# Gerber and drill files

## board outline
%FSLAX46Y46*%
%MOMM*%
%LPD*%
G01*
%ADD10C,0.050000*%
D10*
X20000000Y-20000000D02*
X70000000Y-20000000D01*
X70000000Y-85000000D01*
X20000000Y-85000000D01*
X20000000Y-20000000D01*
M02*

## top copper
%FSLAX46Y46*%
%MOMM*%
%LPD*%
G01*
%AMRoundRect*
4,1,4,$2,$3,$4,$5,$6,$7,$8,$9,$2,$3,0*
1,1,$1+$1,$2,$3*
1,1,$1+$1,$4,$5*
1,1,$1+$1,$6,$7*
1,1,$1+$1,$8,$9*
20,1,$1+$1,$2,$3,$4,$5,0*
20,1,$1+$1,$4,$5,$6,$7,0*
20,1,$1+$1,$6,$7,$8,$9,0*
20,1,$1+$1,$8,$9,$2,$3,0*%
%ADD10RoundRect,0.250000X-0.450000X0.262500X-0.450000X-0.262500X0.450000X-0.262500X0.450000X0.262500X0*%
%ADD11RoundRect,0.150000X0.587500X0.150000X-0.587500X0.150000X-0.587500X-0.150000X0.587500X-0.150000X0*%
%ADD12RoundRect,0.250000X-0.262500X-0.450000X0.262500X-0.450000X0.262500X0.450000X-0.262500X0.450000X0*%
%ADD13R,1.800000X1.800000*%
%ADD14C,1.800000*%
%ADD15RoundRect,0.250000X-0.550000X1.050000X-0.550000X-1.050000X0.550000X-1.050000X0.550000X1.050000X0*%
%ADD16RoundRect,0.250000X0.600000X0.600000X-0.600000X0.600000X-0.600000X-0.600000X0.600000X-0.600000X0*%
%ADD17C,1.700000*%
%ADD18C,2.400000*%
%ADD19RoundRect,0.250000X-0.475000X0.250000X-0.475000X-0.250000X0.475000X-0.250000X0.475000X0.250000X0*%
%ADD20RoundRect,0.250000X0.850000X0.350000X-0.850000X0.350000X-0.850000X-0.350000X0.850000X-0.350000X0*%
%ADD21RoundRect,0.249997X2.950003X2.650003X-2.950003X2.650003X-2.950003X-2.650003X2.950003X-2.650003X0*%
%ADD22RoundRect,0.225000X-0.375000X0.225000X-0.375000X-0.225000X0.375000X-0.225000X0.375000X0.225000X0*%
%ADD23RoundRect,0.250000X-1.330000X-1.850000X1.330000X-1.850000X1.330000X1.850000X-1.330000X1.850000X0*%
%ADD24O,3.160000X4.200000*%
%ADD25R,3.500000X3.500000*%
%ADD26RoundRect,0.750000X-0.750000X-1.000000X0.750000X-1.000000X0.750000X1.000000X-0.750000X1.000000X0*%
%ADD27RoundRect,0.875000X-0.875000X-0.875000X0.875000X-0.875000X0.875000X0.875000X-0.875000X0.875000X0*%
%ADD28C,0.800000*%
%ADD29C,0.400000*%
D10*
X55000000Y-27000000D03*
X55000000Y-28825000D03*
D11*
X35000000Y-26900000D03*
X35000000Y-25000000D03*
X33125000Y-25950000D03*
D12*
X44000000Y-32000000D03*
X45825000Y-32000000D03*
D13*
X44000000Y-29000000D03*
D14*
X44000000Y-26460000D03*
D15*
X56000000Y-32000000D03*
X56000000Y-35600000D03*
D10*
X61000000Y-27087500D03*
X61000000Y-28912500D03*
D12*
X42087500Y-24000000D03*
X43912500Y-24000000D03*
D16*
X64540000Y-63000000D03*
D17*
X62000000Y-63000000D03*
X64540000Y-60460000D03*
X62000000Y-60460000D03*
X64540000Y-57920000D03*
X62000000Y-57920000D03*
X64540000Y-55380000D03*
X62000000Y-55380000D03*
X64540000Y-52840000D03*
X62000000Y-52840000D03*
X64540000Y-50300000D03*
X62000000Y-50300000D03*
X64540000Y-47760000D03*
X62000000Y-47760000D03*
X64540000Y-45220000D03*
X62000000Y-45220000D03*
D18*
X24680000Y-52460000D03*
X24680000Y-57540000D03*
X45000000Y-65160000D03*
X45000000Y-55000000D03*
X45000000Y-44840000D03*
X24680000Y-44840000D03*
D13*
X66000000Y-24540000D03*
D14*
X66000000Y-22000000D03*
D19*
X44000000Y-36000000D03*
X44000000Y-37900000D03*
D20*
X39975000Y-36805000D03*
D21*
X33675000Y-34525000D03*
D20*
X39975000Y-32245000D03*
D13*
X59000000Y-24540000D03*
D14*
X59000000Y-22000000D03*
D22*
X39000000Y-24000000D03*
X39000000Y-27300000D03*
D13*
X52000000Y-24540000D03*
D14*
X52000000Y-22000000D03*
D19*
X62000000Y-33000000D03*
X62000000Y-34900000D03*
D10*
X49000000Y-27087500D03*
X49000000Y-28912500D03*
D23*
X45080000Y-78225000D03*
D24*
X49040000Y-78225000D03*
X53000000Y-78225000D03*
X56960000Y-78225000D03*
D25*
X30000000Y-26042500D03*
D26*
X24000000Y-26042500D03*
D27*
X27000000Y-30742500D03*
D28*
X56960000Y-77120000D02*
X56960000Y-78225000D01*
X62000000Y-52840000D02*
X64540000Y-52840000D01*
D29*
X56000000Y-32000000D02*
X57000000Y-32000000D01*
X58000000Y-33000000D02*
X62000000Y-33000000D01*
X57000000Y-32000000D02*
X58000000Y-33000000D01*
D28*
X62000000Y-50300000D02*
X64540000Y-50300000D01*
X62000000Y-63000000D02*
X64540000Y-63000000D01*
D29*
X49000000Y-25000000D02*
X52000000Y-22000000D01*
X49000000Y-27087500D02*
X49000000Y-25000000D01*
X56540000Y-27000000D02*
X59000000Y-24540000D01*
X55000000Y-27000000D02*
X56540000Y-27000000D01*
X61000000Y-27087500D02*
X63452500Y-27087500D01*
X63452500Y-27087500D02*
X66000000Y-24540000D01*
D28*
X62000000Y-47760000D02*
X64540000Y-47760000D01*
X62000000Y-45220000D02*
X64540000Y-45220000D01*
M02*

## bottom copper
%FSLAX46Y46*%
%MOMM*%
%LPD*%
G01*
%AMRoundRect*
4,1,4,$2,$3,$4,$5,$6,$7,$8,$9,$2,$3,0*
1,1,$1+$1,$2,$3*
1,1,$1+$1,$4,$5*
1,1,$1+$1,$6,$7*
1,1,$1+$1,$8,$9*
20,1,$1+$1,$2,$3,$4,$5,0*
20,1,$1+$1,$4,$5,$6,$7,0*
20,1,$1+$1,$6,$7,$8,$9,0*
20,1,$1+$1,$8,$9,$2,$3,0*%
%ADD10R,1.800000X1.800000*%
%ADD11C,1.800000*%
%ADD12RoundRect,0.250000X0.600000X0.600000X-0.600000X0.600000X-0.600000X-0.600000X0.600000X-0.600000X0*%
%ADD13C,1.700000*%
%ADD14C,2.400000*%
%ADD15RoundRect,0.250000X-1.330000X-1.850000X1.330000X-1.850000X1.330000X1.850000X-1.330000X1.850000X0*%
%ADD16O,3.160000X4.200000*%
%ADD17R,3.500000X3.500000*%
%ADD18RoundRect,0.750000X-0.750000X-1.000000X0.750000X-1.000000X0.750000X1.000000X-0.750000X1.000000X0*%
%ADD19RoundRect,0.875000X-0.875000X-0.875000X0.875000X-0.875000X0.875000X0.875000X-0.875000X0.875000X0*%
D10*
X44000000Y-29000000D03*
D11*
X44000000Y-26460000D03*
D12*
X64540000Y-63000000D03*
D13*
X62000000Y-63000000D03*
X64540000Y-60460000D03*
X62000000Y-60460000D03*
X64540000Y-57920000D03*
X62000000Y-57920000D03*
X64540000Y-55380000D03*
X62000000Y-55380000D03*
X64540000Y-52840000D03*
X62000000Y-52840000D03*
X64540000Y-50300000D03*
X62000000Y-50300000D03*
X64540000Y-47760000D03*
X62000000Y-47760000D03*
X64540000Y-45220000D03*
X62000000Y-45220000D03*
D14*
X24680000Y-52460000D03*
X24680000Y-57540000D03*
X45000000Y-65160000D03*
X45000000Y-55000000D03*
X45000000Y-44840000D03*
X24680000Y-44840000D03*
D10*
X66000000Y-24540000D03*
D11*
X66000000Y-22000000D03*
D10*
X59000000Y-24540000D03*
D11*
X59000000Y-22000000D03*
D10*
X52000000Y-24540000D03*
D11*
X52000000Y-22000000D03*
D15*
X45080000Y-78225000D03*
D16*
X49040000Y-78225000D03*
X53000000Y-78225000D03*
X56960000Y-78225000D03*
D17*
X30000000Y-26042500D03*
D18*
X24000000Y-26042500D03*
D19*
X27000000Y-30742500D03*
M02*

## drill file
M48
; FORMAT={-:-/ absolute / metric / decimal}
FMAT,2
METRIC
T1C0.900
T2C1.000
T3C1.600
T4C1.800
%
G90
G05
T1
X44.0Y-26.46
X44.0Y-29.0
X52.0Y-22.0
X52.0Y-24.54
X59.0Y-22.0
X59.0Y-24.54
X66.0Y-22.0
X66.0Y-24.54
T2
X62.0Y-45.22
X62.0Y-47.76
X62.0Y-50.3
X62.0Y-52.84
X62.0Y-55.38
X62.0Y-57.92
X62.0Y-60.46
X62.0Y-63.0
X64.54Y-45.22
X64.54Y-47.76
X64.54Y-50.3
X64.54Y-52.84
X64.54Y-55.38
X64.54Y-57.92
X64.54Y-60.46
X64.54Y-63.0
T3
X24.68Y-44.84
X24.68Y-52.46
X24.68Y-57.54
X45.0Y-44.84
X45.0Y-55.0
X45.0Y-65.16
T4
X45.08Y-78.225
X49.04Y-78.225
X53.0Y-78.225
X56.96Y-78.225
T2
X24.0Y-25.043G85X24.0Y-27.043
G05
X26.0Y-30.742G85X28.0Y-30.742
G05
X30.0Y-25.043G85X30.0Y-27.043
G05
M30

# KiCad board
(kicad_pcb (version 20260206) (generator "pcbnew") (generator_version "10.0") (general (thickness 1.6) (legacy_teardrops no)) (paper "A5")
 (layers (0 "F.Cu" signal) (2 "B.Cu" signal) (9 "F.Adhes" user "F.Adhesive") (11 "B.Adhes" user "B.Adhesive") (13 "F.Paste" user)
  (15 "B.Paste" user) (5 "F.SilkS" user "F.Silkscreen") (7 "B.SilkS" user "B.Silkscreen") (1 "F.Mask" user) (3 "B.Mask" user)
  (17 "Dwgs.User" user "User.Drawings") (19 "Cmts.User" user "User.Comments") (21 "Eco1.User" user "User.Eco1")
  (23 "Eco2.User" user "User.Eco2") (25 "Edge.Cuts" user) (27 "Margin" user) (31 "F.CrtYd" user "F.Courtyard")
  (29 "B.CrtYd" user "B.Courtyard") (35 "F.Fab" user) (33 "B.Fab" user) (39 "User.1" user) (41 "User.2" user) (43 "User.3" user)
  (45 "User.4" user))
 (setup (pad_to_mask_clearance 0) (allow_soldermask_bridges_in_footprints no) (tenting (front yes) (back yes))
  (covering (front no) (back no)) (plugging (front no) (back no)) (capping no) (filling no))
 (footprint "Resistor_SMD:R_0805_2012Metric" (layer "F.Cu") (at 55 27.9125 -90)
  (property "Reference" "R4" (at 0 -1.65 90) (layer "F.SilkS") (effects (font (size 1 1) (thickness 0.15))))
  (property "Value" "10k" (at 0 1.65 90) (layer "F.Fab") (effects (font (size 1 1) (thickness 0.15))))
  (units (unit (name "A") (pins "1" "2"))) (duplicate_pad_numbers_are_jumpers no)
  (pad "1" smd roundrect (at -0.9125 0 270) (size 1.025 1.4) (layers "F.Cu" "F.Mask" "F.Paste") (roundrect_rratio 0.243902)
   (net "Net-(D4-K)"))
  (pad "2" smd roundrect (at 0.9125 0 270) (size 1.025 1.4) (layers "F.Cu" "F.Mask" "F.Paste") (roundrect_rratio 0.243902) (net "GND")))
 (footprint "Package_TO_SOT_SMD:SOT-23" (layer "F.Cu") (at 34.0625 25.95 180)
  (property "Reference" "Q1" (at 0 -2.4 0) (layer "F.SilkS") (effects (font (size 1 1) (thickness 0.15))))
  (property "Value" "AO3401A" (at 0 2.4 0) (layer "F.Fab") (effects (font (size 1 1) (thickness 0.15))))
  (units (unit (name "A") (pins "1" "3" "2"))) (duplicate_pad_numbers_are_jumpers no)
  (pad "1" smd roundrect (at -0.9375 -0.95 180) (size 1.475 0.6) (layers "F.Cu" "F.Mask" "F.Paste") (roundrect_rratio 0.25)
   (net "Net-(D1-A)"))
  (pad "2" smd roundrect (at -0.9375 0.95 180) (size 1.475 0.6) (layers "F.Cu" "F.Mask" "F.Paste") (roundrect_rratio 0.25)
   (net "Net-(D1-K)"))
  (pad "3" smd roundrect (at 0.9375 0 180) (size 1.475 0.6) (layers "F.Cu" "F.Mask" "F.Paste") (roundrect_rratio 0.25) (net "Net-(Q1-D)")))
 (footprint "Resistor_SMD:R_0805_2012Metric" (layer "F.Cu") (at 44.9125 32)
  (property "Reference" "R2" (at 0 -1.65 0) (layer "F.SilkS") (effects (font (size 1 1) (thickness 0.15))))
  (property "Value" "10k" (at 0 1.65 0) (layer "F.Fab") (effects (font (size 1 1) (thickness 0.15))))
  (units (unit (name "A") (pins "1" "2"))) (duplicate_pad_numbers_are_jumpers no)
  (pad "1" smd roundrect (at -0.9125 0) (size 1.025 1.4) (layers "F.Cu" "F.Mask" "F.Paste") (roundrect_rratio 0.243902) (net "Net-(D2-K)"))
  (pad "2" smd roundrect (at 0.9125 0) (size 1.025 1.4) (layers "F.Cu" "F.Mask" "F.Paste") (roundrect_rratio 0.243902) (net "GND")))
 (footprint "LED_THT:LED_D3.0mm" (layer "F.Cu") (at 44 29 90)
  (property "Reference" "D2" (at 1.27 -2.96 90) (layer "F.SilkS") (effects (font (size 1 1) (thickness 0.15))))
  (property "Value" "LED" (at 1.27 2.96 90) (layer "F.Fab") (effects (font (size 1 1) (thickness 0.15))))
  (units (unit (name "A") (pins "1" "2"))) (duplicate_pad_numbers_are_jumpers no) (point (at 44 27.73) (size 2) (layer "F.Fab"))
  (pad "1" thru_hole rect (at 0 0 90) (size 1.8 1.8) (drill 0.9) (layers "*.Cu" "*.Mask") (remove_unused_layers no) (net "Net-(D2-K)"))
  (pad "2" thru_hole circle (at 2.54 0 90) (size 1.8 1.8) (drill 0.9) (layers "*.Cu" "*.Mask") (remove_unused_layers no) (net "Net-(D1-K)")))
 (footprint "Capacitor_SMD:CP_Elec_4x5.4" (layer "F.Cu") (at 56 33.8 -90)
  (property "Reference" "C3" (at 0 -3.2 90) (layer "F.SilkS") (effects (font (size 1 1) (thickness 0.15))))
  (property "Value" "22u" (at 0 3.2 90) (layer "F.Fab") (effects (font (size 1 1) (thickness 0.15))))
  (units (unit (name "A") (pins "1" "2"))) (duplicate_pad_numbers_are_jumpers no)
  (pad "1" smd roundrect (at -1.8 0 270) (size 2.6 1.6) (layers "F.Cu" "F.Mask" "F.Paste") (roundrect_rratio 0.15625) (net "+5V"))
  (pad "2" smd roundrect (at 1.8 0 270) (size 2.6 1.6) (layers "F.Cu" "F.Mask" "F.Paste") (roundrect_rratio 0.15625) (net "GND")))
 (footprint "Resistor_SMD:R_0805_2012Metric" (layer "F.Cu") (at 61 28 -90)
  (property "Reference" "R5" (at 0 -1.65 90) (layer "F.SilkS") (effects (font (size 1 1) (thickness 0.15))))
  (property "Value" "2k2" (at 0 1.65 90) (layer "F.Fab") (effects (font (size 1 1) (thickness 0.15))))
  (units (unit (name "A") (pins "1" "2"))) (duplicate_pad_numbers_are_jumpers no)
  (pad "1" smd roundrect (at -0.9125 0 270) (size 1.025 1.4) (layers "F.Cu" "F.Mask" "F.Paste") (roundrect_rratio 0.243902)
   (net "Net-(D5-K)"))
  (pad "2" smd roundrect (at 0.9125 0 270) (size 1.025 1.4) (layers "F.Cu" "F.Mask" "F.Paste") (roundrect_rratio 0.243902) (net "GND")))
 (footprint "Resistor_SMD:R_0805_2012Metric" (layer "F.Cu") (at 43 24)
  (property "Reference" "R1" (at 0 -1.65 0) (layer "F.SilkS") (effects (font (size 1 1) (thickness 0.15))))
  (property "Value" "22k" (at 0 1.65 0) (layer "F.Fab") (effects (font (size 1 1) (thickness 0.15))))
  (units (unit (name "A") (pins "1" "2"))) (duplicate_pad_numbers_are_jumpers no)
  (pad "1" smd roundrect (at -0.9125 0) (size 1.025 1.4) (layers "F.Cu" "F.Mask" "F.Paste") (roundrect_rratio 0.243902) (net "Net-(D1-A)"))
  (pad "2" smd roundrect (at 0.9125 0) (size 1.025 1.4) (layers "F.Cu" "F.Mask" "F.Paste") (roundrect_rratio 0.243902) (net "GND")))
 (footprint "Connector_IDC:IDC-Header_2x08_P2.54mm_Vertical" (layer "F.Cu") (at 64.54 63 180)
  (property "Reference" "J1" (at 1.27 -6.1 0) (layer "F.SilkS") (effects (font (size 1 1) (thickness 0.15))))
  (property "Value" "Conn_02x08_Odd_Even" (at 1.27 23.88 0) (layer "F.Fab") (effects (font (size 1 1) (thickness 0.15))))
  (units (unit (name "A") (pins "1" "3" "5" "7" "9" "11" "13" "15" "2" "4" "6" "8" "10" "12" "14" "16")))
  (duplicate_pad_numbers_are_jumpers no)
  (pad "1" thru_hole roundrect (at 0 0 180) (size 1.7 1.7) (drill 1) (layers "*.Cu" "*.Mask") (remove_unused_layers no)
   (roundrect_rratio 0.147059) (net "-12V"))
  (pad "2" thru_hole circle (at 2.54 0 180) (size 1.7 1.7) (drill 1) (layers "*.Cu" "*.Mask") (remove_unused_layers no) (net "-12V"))
  (pad "3" thru_hole circle (at 0 2.54 180) (size 1.7 1.7) (drill 1) (layers "*.Cu" "*.Mask") (remove_unused_layers no) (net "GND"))
  (pad "4" thru_hole circle (at 2.54 2.54 180) (size 1.7 1.7) (drill 1) (layers "*.Cu" "*.Mask") (remove_unused_layers no) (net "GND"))
  (pad "5" thru_hole circle (at 0 5.08 180) (size 1.7 1.7) (drill 1) (layers "*.Cu" "*.Mask") (remove_unused_layers no) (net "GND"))
  (pad "6" thru_hole circle (at 2.54 5.08 180) (size 1.7 1.7) (drill 1) (layers "*.Cu" "*.Mask") (remove_unused_layers no) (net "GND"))
  (pad "7" thru_hole circle (at 0 7.62 180) (size 1.7 1.7) (drill 1) (layers "*.Cu" "*.Mask") (remove_unused_layers no) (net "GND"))
  (pad "8" thru_hole circle (at 2.54 7.62 180) (size 1.7 1.7) (drill 1) (layers "*.Cu" "*.Mask") (remove_unused_layers no) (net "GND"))
  (pad "9" thru_hole circle (at 0 10.16 180) (size 1.7 1.7) (drill 1) (layers "*.Cu" "*.Mask") (remove_unused_layers no) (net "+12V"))
  (pad "10" thru_hole circle (at 2.54 10.16 180) (size 1.7 1.7) (drill 1) (layers "*.Cu" "*.Mask") (remove_unused_layers no) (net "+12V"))
  (pad "11" thru_hole circle (at 0 12.7 180) (size 1.7 1.7) (drill 1) (layers "*.Cu" "*.Mask") (remove_unused_layers no) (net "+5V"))
  (pad "12" thru_hole circle (at 2.54 12.7 180) (size 1.7 1.7) (drill 1) (layers "*.Cu" "*.Mask") (remove_unused_layers no) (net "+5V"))
  (pad "13" thru_hole circle (at 0 15.24 180) (size 1.7 1.7) (drill 1) (layers "*.Cu" "*.Mask") (remove_unused_layers no) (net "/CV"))
  (pad "14" thru_hole circle (at 2.54 15.24 180) (size 1.7 1.7) (drill 1) (layers "*.Cu" "*.Mask") (remove_unused_layers no) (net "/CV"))
  (pad "15" thru_hole circle (at 0 17.78 180) (size 1.7 1.7) (drill 1) (layers "*.Cu" "*.Mask") (remove_unused_layers no) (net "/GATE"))
  (pad "16" thru_hole circle (at 2.54 17.78 180) (size 1.7 1.7) (drill 1) (layers "*.Cu" "*.Mask") (remove_unused_layers no) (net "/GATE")))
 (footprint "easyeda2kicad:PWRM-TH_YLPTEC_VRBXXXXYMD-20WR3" (layer "F.Cu") (at 34.84 55)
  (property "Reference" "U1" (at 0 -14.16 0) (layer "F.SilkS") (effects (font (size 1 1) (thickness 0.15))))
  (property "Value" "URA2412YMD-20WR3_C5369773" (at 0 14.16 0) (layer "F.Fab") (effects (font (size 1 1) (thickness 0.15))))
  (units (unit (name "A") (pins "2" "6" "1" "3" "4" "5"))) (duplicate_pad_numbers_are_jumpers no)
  (pad "1" thru_hole circle (at -10.16 -2.54 90) (size 2.4 2.4) (drill 1.599996) (layers "*.Cu" "*.Mask") (remove_unused_layers no)
   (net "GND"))
  (pad "2" thru_hole circle (at -10.16 2.54 90) (size 2.4 2.4) (drill 1.599996) (layers "*.Cu" "*.Mask") (remove_unused_layers no)
   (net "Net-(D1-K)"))
  (pad "3" thru_hole circle (at 10.16 10.16 90) (size 2.4 2.4) (drill 1.599996) (layers "*.Cu" "*.Mask") (remove_unused_layers no)
   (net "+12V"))
  (pad "4" thru_hole circle (at 10.16 0 90) (size 2.4 2.4) (drill 1.599996) (layers "*.Cu" "*.Mask") (remove_unused_layers no) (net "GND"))
  (pad "5" thru_hole circle (at 10.16 -10.16 90) (size 2.4 2.4) (drill 1.599996) (layers "*.Cu" "*.Mask") (remove_unused_layers no)
   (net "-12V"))
  (pad "6" thru_hole circle (at -10.16 -10.16 90) (size 2.4 2.4) (drill 1.599996) (layers "*.Cu" "*.Mask") (remove_unused_layers no)
   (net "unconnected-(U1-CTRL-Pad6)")))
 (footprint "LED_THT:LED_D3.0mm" (layer "F.Cu") (at 66 24.54 90)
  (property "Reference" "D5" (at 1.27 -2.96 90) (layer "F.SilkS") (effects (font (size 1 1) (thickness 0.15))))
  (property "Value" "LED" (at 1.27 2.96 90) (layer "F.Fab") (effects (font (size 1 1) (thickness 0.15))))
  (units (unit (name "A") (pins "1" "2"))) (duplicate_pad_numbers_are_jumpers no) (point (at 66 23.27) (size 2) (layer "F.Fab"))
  (pad "1" thru_hole rect (at 0 0 90) (size 1.8 1.8) (drill 0.9) (layers "*.Cu" "*.Mask") (remove_unused_layers no) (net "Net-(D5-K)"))
  (pad "2" thru_hole circle (at 2.54 0 90) (size 1.8 1.8) (drill 0.9) (layers "*.Cu" "*.Mask") (remove_unused_layers no) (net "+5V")))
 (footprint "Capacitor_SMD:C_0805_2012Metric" (layer "F.Cu") (at 44 36.95 -90)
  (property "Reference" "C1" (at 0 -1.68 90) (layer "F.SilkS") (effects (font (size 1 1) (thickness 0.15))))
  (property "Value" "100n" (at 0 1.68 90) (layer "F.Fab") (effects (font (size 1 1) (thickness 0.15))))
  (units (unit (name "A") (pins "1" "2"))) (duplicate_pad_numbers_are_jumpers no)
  (pad "1" smd roundrect (at -0.95 0 270) (size 1 1.45) (layers "F.Cu" "F.Mask" "F.Paste") (roundrect_rratio 0.25) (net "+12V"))
  (pad "2" smd roundrect (at 0.95 0 270) (size 1 1.45) (layers "F.Cu" "F.Mask" "F.Paste") (roundrect_rratio 0.25) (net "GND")))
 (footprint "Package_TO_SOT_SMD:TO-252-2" (layer "F.Cu") (at 34.935 34.525 180)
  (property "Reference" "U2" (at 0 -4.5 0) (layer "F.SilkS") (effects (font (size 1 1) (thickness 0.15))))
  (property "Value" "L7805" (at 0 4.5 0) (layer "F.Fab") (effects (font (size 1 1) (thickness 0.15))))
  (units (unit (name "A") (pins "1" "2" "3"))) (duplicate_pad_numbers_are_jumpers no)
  (pad "" smd roundrect (at -0.415 -1.525 180) (size 3.05 2.75) (layers "F.Paste") (roundrect_rratio 0.090909))
  (pad "" smd roundrect (at -0.415 1.525 180) (size 3.05 2.75) (layers "F.Paste") (roundrect_rratio 0.090909))
  (pad "" smd roundrect (at 2.935 -1.525 180) (size 3.05 2.75) (layers "F.Paste") (roundrect_rratio 0.090909))
  (pad "" smd roundrect (at 2.935 1.525 180) (size 3.05 2.75) (layers "F.Paste") (roundrect_rratio 0.090909))
  (pad "1" smd roundrect (at -5.04 -2.28 180) (size 2.2 1.2) (layers "F.Cu" "F.Mask" "F.Paste") (roundrect_rratio 0.208333) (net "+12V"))
  (pad "2" smd roundrect (at 1.26 0 180) (size 6.4 5.8) (layers "F.Cu" "F.Mask") (roundrect_rratio 0.043103) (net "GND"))
  (pad "3" smd roundrect (at -5.04 2.28 180) (size 2.2 1.2) (layers "F.Cu" "F.Mask" "F.Paste") (roundrect_rratio 0.208333) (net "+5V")))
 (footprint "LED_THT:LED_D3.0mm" (layer "F.Cu") (at 59 24.54 90)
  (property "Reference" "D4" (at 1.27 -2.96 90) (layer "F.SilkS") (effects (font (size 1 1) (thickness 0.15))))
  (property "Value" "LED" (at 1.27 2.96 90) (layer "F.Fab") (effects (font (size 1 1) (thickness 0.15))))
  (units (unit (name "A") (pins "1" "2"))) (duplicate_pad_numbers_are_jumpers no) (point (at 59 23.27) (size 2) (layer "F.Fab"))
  (pad "1" thru_hole rect (at 0 0 90) (size 1.8 1.8) (drill 0.9) (layers "*.Cu" "*.Mask") (remove_unused_layers no) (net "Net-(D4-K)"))
  (pad "2" thru_hole circle (at 2.54 0 90) (size 1.8 1.8) (drill 0.9) (layers "*.Cu" "*.Mask") (remove_unused_layers no) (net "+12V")))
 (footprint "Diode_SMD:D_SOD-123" (layer "F.Cu") (at 39 25.65 -90)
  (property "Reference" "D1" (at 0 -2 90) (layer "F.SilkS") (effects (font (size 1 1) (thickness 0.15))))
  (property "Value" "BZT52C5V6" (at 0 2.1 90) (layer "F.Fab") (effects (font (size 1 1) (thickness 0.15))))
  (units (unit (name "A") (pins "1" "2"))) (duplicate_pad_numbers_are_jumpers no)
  (pad "1" smd roundrect (at -1.65 0 270) (size 0.9 1.2) (layers "F.Cu" "F.Mask" "F.Paste") (roundrect_rratio 0.25) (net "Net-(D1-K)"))
  (pad "2" smd roundrect (at 1.65 0 270) (size 0.9 1.2) (layers "F.Cu" "F.Mask" "F.Paste") (roundrect_rratio 0.25) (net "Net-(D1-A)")))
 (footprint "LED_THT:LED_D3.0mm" (layer "F.Cu") (at 52 24.54 90)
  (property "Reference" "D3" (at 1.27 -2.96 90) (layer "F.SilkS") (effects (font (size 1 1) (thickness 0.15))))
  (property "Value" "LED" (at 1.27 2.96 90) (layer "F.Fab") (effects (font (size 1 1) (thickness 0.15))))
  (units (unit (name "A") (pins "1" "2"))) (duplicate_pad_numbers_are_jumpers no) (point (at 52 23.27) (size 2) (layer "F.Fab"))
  (pad "1" thru_hole rect (at 0 0 90) (size 1.8 1.8) (drill 0.9) (layers "*.Cu" "*.Mask") (remove_unused_layers no) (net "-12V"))
  (pad "2" thru_hole circle (at 2.54 0 90) (size 1.8 1.8) (drill 0.9) (layers "*.Cu" "*.Mask") (remove_unused_layers no) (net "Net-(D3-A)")))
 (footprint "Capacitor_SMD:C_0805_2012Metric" (layer "F.Cu") (at 62 33.95 -90)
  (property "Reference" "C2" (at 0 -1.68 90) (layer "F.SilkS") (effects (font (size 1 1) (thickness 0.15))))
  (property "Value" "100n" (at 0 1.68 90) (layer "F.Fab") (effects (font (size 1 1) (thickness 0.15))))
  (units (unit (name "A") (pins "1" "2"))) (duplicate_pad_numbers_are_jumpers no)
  (pad "1" smd roundrect (at -0.95 0 270) (size 1 1.45) (layers "F.Cu" "F.Mask" "F.Paste") (roundrect_rratio 0.25) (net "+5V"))
  (pad "2" smd roundrect (at 0.95 0 270) (size 1 1.45) (layers "F.Cu" "F.Mask" "F.Paste") (roundrect_rratio 0.25) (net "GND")))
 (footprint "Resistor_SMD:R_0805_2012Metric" (layer "F.Cu") (at 49 28 -90)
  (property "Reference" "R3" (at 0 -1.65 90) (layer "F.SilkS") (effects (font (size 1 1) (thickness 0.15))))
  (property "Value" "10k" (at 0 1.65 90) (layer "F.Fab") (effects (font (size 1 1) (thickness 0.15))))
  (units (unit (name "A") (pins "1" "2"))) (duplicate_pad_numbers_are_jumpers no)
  (pad "1" smd roundrect (at -0.9125 0 270) (size 1.025 1.4) (layers "F.Cu" "F.Mask" "F.Paste") (roundrect_rratio 0.243902)
   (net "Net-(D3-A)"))
  (pad "2" smd roundrect (at 0.9125 0 270) (size 1.025 1.4) (layers "F.Cu" "F.Mask" "F.Paste") (roundrect_rratio 0.243902) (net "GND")))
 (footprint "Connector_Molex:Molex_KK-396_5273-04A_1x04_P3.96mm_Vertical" (layer "F.Cu") (at 45.08 78.225)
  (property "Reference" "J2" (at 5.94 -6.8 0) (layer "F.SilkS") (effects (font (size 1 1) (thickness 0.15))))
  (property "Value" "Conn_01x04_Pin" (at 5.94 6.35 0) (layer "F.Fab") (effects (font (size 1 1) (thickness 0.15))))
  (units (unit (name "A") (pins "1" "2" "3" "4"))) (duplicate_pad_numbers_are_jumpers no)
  (pad "1" thru_hole roundrect (at 0 0) (size 3.16 4.2) (drill 1.8) (layers "*.Cu" "*.Mask") (remove_unused_layers no)
   (roundrect_rratio 0.079114) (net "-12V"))
  (pad "2" thru_hole oval (at 3.96 0) (size 3.16 4.2) (drill 1.8) (layers "*.Cu" "*.Mask") (remove_unused_layers no) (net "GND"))
  (pad "3" thru_hole oval (at 7.92 0) (size 3.16 4.2) (drill 1.8) (layers "*.Cu" "*.Mask") (remove_unused_layers no) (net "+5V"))
  (pad "4" thru_hole oval (at 11.88 0) (size 3.16 4.2) (drill 1.8) (layers "*.Cu" "*.Mask") (remove_unused_layers no) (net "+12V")))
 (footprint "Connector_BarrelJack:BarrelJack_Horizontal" (layer "F.Cu") (at 30 26.0425)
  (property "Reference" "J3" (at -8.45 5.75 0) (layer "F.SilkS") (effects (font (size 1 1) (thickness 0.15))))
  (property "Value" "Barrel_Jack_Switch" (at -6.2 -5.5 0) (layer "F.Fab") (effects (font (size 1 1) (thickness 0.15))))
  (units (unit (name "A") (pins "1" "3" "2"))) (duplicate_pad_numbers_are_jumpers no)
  (pad "1" thru_hole rect (at 0 0) (size 3.5 3.5) (drill oval 1 3) (layers "*.Cu" "*.Mask") (remove_unused_layers no) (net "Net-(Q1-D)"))
  (pad "2" thru_hole roundrect (at -6 0) (size 3 3.5) (drill oval 1 3) (layers "*.Cu" "*.Mask") (remove_unused_layers no)
   (roundrect_rratio 0.25) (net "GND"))
  (pad "3" thru_hole roundrect (at -3 4.7) (size 3.5 3.5) (drill oval 3 1) (layers "*.Cu" "*.Mask") (remove_unused_layers no)
   (roundrect_rratio 0.25) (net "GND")))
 (gr_rect (start 20 20) (end 70 85) (stroke (width 0.05) (type solid)) (fill no) (layer "Edge.Cuts"))
 (segment (start 56.96 77.12) (end 56.96 78.225) (width 0.8) (layer "F.Cu") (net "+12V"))
 (segment (start 62 52.84) (end 64.54 52.84) (width 0.8) (layer "F.Cu") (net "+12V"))
 (segment (start 56 32) (end 57 32) (width 0.4) (layer "F.Cu") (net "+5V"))
 (segment (start 58 33) (end 62 33) (width 0.4) (layer "F.Cu") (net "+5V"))
 (segment (start 57 32) (end 58 33) (width 0.4) (layer "F.Cu") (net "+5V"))
 (segment (start 62 50.3) (end 64.54 50.3) (width 0.8) (layer "F.Cu") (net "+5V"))
 (segment (start 62 63) (end 64.54 63) (width 0.8) (layer "F.Cu") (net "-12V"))
 (segment (start 49 25) (end 52 22) (width 0.4) (layer "F.Cu") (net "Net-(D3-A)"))
 (segment (start 49 27.0875) (end 49 25) (width 0.4) (layer "F.Cu") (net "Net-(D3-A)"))
 (segment (start 56.54 27) (end 59 24.54) (width 0.4) (layer "F.Cu") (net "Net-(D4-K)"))
 (segment (start 55 27) (end 56.54 27) (width 0.4) (layer "F.Cu") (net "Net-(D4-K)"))
 (segment (start 61 27.0875) (end 63.4525 27.0875) (width 0.4) (layer "F.Cu") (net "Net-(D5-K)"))
 (segment (start 63.4525 27.0875) (end 66 24.54) (width 0.4) (layer "F.Cu") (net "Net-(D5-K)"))
 (segment (start 62 47.76) (end 64.54 47.76) (width 0.8) (layer "F.Cu") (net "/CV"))
 (segment (start 62 45.22) (end 64.54 45.22) (width 0.8) (layer "F.Cu") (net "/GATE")))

